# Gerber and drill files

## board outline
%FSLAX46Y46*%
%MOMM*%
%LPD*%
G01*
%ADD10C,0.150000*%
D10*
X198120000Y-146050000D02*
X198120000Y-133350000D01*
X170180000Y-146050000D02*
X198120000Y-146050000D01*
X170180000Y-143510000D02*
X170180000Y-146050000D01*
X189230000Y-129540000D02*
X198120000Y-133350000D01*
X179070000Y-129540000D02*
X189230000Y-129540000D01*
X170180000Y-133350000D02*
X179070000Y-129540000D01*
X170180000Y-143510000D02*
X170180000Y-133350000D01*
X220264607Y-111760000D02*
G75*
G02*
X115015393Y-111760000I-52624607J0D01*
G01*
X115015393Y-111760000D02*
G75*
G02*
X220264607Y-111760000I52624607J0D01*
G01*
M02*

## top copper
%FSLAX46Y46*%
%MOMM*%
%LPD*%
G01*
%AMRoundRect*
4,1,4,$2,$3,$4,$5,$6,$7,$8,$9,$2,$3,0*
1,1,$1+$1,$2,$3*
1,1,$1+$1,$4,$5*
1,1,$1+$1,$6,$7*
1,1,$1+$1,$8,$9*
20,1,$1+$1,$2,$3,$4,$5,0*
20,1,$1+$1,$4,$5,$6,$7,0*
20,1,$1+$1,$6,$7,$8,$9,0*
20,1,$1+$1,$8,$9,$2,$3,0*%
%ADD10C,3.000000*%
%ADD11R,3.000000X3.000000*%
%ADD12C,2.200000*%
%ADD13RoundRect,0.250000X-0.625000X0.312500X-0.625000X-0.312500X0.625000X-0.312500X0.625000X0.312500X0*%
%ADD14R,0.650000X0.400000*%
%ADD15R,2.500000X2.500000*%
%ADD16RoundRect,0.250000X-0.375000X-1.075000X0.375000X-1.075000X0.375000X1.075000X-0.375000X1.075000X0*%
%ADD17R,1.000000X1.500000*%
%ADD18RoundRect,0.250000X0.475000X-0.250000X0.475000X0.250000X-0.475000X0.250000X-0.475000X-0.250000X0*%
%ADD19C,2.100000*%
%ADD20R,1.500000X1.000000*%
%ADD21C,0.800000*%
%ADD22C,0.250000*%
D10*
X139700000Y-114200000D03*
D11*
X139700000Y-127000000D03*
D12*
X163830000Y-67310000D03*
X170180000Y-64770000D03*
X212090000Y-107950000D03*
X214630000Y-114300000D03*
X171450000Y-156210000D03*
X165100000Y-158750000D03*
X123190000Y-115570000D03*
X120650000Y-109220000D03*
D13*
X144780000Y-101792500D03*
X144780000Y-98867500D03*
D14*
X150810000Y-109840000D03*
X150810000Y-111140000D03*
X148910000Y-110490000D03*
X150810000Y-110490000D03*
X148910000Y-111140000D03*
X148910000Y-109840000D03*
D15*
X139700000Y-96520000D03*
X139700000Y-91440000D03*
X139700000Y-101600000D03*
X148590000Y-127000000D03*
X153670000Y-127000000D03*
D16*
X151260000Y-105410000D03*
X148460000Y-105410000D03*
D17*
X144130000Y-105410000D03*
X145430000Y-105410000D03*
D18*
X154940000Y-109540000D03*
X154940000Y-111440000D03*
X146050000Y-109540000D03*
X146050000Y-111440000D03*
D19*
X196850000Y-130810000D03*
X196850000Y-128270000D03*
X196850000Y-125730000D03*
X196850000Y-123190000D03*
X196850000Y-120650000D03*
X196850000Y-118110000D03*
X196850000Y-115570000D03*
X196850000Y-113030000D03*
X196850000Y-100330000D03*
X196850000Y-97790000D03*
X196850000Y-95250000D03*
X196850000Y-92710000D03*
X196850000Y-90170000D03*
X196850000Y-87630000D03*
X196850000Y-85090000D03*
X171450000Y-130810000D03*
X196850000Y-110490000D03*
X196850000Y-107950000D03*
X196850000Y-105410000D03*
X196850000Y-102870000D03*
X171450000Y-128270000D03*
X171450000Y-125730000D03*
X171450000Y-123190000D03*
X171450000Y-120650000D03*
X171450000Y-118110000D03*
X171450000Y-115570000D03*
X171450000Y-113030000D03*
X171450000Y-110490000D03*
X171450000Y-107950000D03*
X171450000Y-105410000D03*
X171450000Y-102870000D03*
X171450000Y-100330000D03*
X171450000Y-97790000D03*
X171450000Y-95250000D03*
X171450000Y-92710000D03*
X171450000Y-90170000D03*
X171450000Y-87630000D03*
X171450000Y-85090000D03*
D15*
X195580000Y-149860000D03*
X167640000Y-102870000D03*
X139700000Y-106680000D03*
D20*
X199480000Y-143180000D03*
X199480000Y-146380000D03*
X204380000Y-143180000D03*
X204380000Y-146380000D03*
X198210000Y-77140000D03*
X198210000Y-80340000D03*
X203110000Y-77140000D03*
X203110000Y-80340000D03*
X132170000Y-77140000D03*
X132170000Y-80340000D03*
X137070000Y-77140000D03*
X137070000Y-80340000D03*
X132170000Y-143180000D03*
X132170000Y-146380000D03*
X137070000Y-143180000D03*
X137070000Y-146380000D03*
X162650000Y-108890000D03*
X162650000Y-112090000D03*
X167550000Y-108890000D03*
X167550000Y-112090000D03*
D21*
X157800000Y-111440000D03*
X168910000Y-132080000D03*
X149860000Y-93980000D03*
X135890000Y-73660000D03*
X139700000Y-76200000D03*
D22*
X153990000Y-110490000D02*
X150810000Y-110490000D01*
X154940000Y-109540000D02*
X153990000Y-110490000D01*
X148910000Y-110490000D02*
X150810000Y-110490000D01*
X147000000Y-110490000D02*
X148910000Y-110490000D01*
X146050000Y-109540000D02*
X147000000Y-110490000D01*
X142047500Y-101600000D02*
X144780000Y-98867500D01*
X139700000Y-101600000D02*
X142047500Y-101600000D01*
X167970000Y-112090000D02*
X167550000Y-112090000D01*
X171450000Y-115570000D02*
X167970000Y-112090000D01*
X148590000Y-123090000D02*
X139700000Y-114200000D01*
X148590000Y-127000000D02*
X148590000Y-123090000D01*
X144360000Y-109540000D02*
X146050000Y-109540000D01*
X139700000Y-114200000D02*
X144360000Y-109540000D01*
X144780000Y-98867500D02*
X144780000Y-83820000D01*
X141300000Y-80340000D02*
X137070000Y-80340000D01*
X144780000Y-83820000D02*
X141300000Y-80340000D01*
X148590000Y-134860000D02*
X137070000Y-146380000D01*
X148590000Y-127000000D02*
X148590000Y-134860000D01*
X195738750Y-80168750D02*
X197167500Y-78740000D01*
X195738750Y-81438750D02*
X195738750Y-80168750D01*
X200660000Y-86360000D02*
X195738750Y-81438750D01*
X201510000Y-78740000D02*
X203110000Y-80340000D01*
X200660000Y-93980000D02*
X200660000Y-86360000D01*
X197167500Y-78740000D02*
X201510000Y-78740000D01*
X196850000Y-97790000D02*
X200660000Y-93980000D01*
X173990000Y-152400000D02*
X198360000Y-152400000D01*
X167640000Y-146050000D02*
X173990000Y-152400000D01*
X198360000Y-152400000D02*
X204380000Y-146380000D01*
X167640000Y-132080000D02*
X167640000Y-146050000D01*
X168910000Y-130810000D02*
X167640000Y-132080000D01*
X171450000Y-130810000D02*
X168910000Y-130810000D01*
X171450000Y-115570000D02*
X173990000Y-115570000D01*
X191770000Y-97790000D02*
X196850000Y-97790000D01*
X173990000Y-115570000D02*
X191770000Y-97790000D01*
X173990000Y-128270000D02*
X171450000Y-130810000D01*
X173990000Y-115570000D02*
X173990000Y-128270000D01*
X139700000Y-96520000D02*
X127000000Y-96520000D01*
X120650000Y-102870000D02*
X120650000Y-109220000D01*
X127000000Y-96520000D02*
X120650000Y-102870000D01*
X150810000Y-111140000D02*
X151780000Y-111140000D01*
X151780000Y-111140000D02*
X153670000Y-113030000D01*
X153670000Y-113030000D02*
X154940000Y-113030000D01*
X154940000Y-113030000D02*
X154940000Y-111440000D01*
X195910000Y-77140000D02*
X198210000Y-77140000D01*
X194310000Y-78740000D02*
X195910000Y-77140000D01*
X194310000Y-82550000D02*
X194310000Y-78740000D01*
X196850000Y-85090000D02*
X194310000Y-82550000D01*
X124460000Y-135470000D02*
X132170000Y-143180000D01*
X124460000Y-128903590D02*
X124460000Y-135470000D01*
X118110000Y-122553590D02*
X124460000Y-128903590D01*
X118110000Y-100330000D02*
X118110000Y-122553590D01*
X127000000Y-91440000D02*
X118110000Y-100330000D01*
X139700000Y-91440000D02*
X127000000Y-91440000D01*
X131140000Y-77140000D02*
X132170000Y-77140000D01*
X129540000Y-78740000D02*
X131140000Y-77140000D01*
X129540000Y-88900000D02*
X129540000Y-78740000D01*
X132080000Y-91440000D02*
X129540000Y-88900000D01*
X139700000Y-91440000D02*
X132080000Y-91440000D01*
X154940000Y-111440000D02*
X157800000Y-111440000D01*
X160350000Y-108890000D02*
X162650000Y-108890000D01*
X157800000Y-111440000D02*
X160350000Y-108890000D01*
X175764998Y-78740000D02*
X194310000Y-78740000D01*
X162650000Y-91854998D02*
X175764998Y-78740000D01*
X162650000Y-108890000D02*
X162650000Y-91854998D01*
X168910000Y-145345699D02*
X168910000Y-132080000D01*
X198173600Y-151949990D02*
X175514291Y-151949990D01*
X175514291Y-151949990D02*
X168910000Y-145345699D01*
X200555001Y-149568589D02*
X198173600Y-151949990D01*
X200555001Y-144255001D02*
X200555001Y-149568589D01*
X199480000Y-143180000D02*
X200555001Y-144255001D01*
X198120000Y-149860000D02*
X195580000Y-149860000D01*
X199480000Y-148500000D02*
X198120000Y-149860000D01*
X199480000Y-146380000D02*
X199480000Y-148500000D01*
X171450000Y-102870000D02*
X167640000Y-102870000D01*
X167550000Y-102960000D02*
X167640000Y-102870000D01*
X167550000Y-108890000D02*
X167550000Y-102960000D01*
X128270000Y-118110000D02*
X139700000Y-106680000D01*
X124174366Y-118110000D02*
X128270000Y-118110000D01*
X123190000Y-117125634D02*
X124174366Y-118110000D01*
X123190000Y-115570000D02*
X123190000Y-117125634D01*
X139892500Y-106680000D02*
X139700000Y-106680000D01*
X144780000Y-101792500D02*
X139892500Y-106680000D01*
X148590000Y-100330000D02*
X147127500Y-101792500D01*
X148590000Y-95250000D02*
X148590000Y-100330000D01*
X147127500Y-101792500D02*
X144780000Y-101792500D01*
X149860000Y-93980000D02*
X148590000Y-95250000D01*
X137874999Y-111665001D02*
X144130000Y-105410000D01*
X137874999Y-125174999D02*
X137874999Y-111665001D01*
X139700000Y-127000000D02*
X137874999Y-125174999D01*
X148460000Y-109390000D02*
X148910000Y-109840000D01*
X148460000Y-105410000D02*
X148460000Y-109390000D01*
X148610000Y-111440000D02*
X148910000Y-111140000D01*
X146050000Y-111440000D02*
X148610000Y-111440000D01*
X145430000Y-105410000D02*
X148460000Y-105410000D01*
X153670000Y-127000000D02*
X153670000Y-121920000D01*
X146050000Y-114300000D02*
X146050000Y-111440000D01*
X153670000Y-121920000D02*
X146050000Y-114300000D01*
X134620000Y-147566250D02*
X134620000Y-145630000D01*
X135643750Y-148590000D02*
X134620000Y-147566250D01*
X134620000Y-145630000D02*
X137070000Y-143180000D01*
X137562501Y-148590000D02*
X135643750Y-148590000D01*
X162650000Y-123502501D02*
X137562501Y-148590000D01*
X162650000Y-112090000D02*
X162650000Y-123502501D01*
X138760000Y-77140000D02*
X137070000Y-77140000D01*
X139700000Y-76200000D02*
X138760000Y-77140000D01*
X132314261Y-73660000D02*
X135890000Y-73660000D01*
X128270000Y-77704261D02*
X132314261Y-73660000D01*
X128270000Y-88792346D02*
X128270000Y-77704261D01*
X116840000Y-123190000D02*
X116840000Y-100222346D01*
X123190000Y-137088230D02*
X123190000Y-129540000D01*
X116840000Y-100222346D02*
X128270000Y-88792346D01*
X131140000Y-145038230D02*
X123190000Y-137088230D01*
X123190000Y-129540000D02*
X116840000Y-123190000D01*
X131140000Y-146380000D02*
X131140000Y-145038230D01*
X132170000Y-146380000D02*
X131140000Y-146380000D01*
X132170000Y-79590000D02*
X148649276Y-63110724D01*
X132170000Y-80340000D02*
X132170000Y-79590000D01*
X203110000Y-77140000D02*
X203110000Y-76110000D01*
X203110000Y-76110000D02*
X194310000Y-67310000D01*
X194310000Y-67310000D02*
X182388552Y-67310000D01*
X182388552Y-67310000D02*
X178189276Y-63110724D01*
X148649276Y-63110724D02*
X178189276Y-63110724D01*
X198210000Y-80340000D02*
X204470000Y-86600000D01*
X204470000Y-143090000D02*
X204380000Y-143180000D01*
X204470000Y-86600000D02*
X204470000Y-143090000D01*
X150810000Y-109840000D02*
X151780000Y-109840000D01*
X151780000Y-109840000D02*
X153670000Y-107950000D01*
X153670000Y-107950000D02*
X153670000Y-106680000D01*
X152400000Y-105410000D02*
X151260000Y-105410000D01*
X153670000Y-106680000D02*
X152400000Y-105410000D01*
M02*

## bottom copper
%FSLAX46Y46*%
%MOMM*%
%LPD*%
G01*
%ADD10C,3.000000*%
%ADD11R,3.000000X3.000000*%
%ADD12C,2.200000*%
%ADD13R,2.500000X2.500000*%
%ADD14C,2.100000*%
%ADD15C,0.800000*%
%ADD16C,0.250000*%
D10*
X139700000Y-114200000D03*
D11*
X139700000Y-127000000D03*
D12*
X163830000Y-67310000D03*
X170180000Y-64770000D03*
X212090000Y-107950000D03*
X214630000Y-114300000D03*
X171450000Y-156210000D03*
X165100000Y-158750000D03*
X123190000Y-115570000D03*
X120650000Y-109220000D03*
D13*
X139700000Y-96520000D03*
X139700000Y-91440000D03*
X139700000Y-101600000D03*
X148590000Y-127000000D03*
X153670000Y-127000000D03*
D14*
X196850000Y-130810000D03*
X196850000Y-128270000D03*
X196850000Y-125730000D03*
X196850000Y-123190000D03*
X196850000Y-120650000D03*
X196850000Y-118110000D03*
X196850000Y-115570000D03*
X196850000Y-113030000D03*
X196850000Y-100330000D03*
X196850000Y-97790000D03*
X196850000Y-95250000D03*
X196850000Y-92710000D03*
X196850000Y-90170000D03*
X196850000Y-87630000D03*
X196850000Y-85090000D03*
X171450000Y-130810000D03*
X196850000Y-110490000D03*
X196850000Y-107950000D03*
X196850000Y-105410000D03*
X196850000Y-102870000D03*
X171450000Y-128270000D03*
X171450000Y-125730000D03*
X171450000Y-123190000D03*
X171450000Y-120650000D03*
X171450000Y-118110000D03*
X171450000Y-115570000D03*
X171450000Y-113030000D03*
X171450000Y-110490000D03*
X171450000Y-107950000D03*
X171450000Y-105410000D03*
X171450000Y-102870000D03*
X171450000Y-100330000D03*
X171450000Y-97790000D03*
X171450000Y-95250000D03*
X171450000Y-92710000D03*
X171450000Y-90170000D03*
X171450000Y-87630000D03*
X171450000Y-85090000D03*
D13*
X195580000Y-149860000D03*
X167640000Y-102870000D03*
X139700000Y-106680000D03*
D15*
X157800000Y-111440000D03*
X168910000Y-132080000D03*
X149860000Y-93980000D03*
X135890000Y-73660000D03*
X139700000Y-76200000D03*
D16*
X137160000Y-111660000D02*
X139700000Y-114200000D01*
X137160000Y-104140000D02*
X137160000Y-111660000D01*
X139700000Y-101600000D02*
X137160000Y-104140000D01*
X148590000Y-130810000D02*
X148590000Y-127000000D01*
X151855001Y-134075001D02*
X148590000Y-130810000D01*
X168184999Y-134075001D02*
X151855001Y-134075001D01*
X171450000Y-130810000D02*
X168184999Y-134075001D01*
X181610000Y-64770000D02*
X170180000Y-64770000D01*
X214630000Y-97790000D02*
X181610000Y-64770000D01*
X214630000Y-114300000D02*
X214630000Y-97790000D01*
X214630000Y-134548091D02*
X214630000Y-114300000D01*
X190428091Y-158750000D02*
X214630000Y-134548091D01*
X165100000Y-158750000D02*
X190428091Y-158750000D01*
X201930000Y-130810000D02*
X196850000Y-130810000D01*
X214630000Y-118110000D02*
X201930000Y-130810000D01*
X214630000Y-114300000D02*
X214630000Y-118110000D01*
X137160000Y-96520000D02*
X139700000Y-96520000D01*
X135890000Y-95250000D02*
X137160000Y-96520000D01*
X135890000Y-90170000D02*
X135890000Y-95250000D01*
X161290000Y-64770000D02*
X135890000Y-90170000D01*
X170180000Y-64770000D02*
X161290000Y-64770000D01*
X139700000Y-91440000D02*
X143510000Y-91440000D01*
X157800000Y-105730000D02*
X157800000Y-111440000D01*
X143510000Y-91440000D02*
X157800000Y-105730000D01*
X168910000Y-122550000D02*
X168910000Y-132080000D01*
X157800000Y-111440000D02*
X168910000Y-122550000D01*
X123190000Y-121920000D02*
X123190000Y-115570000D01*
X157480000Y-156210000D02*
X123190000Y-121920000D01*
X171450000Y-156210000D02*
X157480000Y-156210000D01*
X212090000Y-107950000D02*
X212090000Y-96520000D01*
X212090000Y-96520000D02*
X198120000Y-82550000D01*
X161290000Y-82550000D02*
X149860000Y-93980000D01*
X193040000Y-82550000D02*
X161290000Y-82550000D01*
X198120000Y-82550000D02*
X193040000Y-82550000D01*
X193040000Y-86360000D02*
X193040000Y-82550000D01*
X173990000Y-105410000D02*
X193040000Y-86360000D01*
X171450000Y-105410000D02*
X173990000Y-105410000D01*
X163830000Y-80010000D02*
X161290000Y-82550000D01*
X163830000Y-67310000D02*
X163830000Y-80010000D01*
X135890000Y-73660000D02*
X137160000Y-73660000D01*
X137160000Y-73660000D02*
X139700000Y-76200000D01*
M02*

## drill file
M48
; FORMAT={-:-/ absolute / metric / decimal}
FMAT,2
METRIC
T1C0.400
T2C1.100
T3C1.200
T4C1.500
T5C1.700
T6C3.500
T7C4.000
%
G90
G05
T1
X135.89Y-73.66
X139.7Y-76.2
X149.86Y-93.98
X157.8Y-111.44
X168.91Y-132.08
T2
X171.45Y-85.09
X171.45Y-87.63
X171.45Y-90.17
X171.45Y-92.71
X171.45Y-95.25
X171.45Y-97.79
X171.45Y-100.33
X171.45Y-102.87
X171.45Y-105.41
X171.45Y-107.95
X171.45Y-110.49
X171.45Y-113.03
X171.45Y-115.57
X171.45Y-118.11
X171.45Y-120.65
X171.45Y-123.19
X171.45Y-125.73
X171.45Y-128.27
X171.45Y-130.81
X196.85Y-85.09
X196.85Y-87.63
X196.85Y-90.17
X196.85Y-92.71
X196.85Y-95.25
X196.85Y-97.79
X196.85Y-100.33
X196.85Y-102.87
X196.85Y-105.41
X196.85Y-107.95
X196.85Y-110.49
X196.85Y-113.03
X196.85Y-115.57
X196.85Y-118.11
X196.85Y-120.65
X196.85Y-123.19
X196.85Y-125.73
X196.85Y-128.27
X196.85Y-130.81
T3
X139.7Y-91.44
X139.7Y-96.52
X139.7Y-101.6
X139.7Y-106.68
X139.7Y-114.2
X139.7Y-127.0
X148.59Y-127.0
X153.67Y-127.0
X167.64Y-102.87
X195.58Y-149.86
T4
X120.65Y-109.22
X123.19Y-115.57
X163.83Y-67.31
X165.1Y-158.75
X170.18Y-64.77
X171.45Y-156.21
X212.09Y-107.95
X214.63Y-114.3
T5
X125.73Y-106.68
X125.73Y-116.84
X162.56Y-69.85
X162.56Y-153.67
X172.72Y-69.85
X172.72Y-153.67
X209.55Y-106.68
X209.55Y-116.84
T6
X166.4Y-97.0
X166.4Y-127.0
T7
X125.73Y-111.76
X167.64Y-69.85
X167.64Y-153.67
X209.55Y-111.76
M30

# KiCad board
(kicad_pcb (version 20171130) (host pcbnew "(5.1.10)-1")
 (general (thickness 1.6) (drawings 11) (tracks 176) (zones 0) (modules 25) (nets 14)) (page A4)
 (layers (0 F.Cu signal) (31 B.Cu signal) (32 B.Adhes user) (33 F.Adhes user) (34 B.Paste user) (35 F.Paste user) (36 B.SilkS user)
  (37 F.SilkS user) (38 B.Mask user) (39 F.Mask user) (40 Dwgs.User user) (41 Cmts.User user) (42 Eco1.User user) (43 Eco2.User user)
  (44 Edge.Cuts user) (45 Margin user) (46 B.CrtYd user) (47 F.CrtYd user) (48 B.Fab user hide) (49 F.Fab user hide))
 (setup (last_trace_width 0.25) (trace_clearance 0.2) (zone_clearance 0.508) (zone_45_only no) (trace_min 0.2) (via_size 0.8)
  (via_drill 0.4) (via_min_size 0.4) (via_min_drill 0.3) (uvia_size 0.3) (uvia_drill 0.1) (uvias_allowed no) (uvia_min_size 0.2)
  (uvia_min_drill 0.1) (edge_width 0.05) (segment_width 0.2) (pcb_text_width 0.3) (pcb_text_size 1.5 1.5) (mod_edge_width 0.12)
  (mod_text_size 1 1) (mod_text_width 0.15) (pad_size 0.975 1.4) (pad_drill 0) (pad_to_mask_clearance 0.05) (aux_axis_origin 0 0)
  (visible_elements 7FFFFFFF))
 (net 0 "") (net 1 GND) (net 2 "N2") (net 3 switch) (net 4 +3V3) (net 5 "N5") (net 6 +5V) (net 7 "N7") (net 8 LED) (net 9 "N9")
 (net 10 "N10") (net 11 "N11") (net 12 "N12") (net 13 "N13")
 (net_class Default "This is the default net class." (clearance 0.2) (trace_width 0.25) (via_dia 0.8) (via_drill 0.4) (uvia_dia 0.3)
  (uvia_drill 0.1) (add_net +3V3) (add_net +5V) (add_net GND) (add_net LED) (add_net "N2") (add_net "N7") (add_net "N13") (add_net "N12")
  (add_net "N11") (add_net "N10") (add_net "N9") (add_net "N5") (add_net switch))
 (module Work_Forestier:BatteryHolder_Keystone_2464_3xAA (layer B.Cu) (at 139.7 127)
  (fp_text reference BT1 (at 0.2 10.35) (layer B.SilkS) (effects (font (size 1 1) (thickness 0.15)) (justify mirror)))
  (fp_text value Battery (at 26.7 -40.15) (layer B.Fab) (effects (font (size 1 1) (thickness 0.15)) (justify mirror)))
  (pad "" np_thru_hole circle (at 26.7 -30) (size 3.5 3.5) (drill 3.5) (layers *.Cu *.Mask))
  (pad "" np_thru_hole circle (at 26.7 0) (size 3.5 3.5) (drill 3.5) (layers *.Cu *.Mask))
  (pad 2 thru_hole circle (at 0 -12.8) (size 3 3) (drill 1.2) (layers *.Cu *.Mask) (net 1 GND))
  (pad 1 thru_hole rect (at 0 0) (size 3 3) (drill 1.2) (layers *.Cu *.Mask) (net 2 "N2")))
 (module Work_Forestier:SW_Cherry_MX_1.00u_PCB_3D (layer F.Cu) (at 170.18 64.77)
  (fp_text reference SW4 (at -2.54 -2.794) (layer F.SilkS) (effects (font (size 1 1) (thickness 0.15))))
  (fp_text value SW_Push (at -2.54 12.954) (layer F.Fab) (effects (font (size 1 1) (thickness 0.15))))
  (pad "" np_thru_hole circle (at 2.54 5.08) (size 1.7 1.7) (drill 1.7) (layers *.Cu *.Mask))
  (pad "" np_thru_hole circle (at -7.62 5.08) (size 1.7 1.7) (drill 1.7) (layers *.Cu *.Mask))
  (pad "" np_thru_hole circle (at -2.54 5.08) (size 4 4) (drill 4) (layers *.Cu *.Mask))
  (pad 2 thru_hole circle (at -6.35 2.54) (size 2.2 2.2) (drill 1.5) (layers *.Cu *.Mask) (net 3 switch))
  (pad 1 thru_hole circle (at 0 0) (size 2.2 2.2) (drill 1.5) (layers *.Cu *.Mask) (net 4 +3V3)))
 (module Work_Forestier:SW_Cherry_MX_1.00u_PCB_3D (layer F.Cu) (at 214.63 114.3 270)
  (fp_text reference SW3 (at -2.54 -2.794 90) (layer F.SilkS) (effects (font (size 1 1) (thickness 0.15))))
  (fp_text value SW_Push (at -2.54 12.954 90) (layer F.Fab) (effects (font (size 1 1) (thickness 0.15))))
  (pad "" np_thru_hole circle (at 2.54 5.08 270) (size 1.7 1.7) (drill 1.7) (layers *.Cu *.Mask))
  (pad "" np_thru_hole circle (at -7.62 5.08 270) (size 1.7 1.7) (drill 1.7) (layers *.Cu *.Mask))
  (pad "" np_thru_hole circle (at -2.54 5.08 270) (size 4 4) (drill 4) (layers *.Cu *.Mask))
  (pad 2 thru_hole circle (at -6.35 2.54 270) (size 2.2 2.2) (drill 1.5) (layers *.Cu *.Mask) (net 3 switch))
  (pad 1 thru_hole circle (at 0 0 270) (size 2.2 2.2) (drill 1.5) (layers *.Cu *.Mask) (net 4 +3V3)))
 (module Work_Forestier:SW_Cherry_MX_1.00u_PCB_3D (layer F.Cu) (at 165.1 158.75 180)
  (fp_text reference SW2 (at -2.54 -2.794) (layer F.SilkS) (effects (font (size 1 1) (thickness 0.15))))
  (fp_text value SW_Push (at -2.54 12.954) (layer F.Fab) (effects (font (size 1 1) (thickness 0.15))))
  (pad "" np_thru_hole circle (at 2.54 5.08 180) (size 1.7 1.7) (drill 1.7) (layers *.Cu *.Mask))
  (pad "" np_thru_hole circle (at -7.62 5.08 180) (size 1.7 1.7) (drill 1.7) (layers *.Cu *.Mask))
  (pad "" np_thru_hole circle (at -2.54 5.08 180) (size 4 4) (drill 4) (layers *.Cu *.Mask))
  (pad 2 thru_hole circle (at -6.35 2.54 180) (size 2.2 2.2) (drill 1.5) (layers *.Cu *.Mask) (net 3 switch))
  (pad 1 thru_hole circle (at 0 0 180) (size 2.2 2.2) (drill 1.5) (layers *.Cu *.Mask) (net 4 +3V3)))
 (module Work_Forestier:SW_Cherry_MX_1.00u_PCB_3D (layer F.Cu) (at 120.65 109.22 90)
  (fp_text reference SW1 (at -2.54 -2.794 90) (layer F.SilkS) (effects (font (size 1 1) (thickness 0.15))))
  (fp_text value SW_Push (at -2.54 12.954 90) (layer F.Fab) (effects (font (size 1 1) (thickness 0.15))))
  (pad "" np_thru_hole circle (at 2.54 5.08 90) (size 1.7 1.7) (drill 1.7) (layers *.Cu *.Mask))
  (pad "" np_thru_hole circle (at -7.62 5.08 90) (size 1.7 1.7) (drill 1.7) (layers *.Cu *.Mask))
  (pad "" np_thru_hole circle (at -2.54 5.08 90) (size 4 4) (drill 4) (layers *.Cu *.Mask))
  (pad 2 thru_hole circle (at -6.35 2.54 90) (size 2.2 2.2) (drill 1.5) (layers *.Cu *.Mask) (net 3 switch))
  (pad 1 thru_hole circle (at 0 0 90) (size 2.2 2.2) (drill 1.5) (layers *.Cu *.Mask) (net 4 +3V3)))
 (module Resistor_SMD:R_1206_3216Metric (layer F.Cu) (at 144.78 100.33 270)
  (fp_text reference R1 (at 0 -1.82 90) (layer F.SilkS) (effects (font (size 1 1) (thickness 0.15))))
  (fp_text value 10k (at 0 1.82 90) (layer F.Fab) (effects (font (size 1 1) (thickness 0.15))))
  (pad 2 smd roundrect (at 1.4625 0 270) (size 1.125 1.75) (layers F.Cu F.Paste F.Mask) (roundrect_rratio 0.222222) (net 3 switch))
  (pad 1 smd roundrect (at -1.4625 0 270) (size 1.125 1.75) (layers F.Cu F.Paste F.Mask) (roundrect_rratio 0.222222) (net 1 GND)))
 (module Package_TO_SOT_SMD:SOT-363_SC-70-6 (layer F.Cu) (at 149.86 110.49)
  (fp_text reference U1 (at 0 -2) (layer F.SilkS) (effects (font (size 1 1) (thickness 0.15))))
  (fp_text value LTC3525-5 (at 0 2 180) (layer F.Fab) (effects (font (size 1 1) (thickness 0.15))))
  (pad 6 smd rect (at 0.95 -0.65) (size 0.65 0.4) (layers F.Cu F.Paste F.Mask) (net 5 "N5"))
  (pad 4 smd rect (at 0.95 0.65) (size 0.65 0.4) (layers F.Cu F.Paste F.Mask) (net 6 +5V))
  (pad 2 smd rect (at -0.95 0) (size 0.65 0.4) (layers F.Cu F.Paste F.Mask) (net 1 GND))
  (pad 5 smd rect (at 0.95 0) (size 0.65 0.4) (layers F.Cu F.Paste F.Mask) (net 1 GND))
  (pad 3 smd rect (at -0.95 0.65) (size 0.65 0.4) (layers F.Cu F.Paste F.Mask) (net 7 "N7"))
  (pad 1 smd rect (at -0.95 -0.65) (size 0.65 0.4) (layers F.Cu F.Paste F.Mask) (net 7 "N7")))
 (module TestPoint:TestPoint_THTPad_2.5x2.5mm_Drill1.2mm (layer F.Cu) (at 139.7 96.52)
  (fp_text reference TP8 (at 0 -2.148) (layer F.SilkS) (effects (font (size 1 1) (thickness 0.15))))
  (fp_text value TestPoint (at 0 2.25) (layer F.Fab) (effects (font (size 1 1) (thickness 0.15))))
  (pad 1 thru_hole rect (at 0 0) (size 2.5 2.5) (drill 1.2) (layers *.Cu *.Mask) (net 4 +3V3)))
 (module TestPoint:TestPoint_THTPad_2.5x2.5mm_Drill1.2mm (layer F.Cu) (at 139.7 91.44)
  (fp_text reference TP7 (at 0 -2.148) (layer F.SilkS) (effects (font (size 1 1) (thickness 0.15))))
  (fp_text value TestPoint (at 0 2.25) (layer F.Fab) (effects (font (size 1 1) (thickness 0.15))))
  (pad 1 thru_hole rect (at 0 0) (size 2.5 2.5) (drill 1.2) (layers *.Cu *.Mask) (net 6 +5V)))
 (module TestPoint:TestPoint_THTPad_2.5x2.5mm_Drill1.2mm (layer F.Cu) (at 139.7 101.6)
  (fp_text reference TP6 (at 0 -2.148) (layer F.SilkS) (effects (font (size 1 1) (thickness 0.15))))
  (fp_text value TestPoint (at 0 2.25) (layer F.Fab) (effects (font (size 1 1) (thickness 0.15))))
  (pad 1 thru_hole rect (at 0 0) (size 2.5 2.5) (drill 1.2) (layers *.Cu *.Mask) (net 1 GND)))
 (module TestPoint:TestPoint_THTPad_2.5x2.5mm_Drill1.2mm (layer F.Cu) (at 148.59 127)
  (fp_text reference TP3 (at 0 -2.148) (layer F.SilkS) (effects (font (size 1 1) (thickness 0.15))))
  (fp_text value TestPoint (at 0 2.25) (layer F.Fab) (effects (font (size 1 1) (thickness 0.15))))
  (pad 1 thru_hole rect (at 0 0) (size 2.5 2.5) (drill 1.2) (layers *.Cu *.Mask) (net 1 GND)))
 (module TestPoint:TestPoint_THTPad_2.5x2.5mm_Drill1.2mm (layer F.Cu) (at 153.67 127)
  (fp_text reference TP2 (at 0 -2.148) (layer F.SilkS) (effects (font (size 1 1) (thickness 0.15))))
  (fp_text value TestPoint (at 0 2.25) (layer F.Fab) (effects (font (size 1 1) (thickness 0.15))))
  (pad 1 thru_hole rect (at 0 0) (size 2.5 2.5) (drill 1.2) (layers *.Cu *.Mask) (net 7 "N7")))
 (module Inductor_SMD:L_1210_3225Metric (layer F.Cu) (at 149.86 105.41)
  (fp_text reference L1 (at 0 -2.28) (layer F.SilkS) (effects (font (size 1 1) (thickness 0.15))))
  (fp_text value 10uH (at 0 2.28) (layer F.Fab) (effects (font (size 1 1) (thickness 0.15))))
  (pad 2 smd roundrect (at 1.4 0) (size 1.25 2.65) (layers F.Cu F.Paste F.Mask) (roundrect_rratio 0.2) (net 5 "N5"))
  (pad 1 smd roundrect (at -1.4 0) (size 1.25 2.65) (layers F.Cu F.Paste F.Mask) (roundrect_rratio 0.2) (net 7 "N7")))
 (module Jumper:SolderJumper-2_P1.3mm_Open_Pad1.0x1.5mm (layer F.Cu) (at 144.78 105.41)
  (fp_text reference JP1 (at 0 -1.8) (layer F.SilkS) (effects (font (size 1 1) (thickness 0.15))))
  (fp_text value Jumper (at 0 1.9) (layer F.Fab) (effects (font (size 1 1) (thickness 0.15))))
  (pad 1 smd rect (at -0.65 0) (size 1 1.5) (layers F.Cu F.Mask) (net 2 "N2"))
  (pad 2 smd rect (at 0.65 0) (size 1 1.5) (layers F.Cu F.Mask) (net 7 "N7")))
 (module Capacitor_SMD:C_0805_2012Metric (layer F.Cu) (at 154.94 110.49 90)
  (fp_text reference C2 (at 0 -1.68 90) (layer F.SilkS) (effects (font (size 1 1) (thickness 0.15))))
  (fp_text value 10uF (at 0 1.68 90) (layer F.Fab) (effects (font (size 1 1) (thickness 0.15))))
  (pad 2 smd roundrect (at 0.95 0 90) (size 1 1.45) (layers F.Cu F.Paste F.Mask) (roundrect_rratio 0.25) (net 1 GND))
  (pad 1 smd roundrect (at -0.95 0 90) (size 1 1.45) (layers F.Cu F.Paste F.Mask) (roundrect_rratio 0.25) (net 6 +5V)))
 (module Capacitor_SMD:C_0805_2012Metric (layer F.Cu) (at 146.05 110.49 90)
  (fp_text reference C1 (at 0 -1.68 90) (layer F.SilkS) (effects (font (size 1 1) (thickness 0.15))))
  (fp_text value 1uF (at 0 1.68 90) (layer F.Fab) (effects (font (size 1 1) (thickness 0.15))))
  (pad 2 smd roundrect (at 0.95 0 90) (size 1 1.45) (layers F.Cu F.Paste F.Mask) (roundrect_rratio 0.25) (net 1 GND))
  (pad 1 smd roundrect (at -0.95 0 90) (size 1 1.45) (layers F.Cu F.Paste F.Mask) (roundrect_rratio 0.25) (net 7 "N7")))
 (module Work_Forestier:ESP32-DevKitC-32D (layer F.Cu) (at 198.12 139.7 90)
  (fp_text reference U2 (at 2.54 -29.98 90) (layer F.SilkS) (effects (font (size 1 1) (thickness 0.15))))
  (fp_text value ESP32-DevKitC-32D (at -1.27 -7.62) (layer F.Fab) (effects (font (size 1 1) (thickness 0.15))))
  (pad 3V3 thru_hole circle (at 8.89 -1.27 90) (size 2.1 2.1) (drill 1.1) (layers *.Cu *.Mask) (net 4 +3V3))
  (pad EN thru_hole circle (at 11.43 -1.27 90) (size 2.1 2.1) (drill 1.1) (layers *.Cu *.Mask))
  (pad SVP thru_hole circle (at 13.97 -1.27 90) (size 2.1 2.1) (drill 1.1) (layers *.Cu *.Mask))
  (pad SVN thru_hole circle (at 16.51 -1.27 90) (size 2.1 2.1) (drill 1.1) (layers *.Cu *.Mask))
  (pad IO34 thru_hole circle (at 19.05 -1.27 90) (size 2.1 2.1) (drill 1.1) (layers *.Cu *.Mask))
  (pad IO35 thru_hole circle (at 21.59 -1.27 90) (size 2.1 2.1) (drill 1.1) (layers *.Cu *.Mask))
  (pad IO32 thru_hole circle (at 24.13 -1.27 90) (size 2.1 2.1) (drill 1.1) (layers *.Cu *.Mask))
  (pad IO33 thru_hole circle (at 26.67 -1.27 90) (size 2.1 2.1) (drill 1.1) (layers *.Cu *.Mask))
  (pad IO12 thru_hole circle (at 39.37 -1.27 90) (size 2.1 2.1) (drill 1.1) (layers *.Cu *.Mask))
  (pad GND0 thru_hole circle (at 41.91 -1.27 90) (size 2.1 2.1) (drill 1.1) (layers *.Cu *.Mask) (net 1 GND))
  (pad IO13 thru_hole circle (at 44.45 -1.27 90) (size 2.1 2.1) (drill 1.1) (layers *.Cu *.Mask))
  (pad SD2 thru_hole circle (at 46.99 -1.27 90) (size 2.1 2.1) (drill 1.1) (layers *.Cu *.Mask))
  (pad SD3 thru_hole circle (at 49.53 -1.27 90) (size 2.1 2.1) (drill 1.1) (layers *.Cu *.Mask))
  (pad CMD thru_hole circle (at 52.07 -1.27 90) (size 2.1 2.1) (drill 1.1) (layers *.Cu *.Mask))
  (pad 5V thru_hole circle (at 54.61 -1.27 90) (size 2.1 2.1) (drill 1.1) (layers *.Cu *.Mask) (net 6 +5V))
  (pad GND1 thru_hole circle (at 8.89 -26.67 90) (size 2.1 2.1) (drill 1.1) (layers *.Cu *.Mask) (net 1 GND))
  (pad IO25 thru_hole circle (at 29.21 -1.27 90) (size 2.1 2.1) (drill 1.1) (layers *.Cu *.Mask))
  (pad IO26 thru_hole circle (at 31.75 -1.27 90) (size 2.1 2.1) (drill 1.1) (layers *.Cu *.Mask))
  (pad IO27 thru_hole circle (at 34.29 -1.27 90) (size 2.1 2.1) (drill 1.1) (layers *.Cu *.Mask))
  (pad IO14 thru_hole circle (at 36.83 -1.27 90) (size 2.1 2.1) (drill 1.1) (layers *.Cu *.Mask))
  (pad IO23 thru_hole circle (at 11.43 -26.67 90) (size 2.1 2.1) (drill 1.1) (layers *.Cu *.Mask))
  (pad IO22 thru_hole circle (at 13.97 -26.67 90) (size 2.1 2.1) (drill 1.1) (layers *.Cu *.Mask))
  (pad TXD0 thru_hole circle (at 16.51 -26.67 90) (size 2.1 2.1) (drill 1.1) (layers *.Cu *.Mask))
  (pad RXD0 thru_hole circle (at 19.05 -26.67 90) (size 2.1 2.1) (drill 1.1) (layers *.Cu *.Mask))
  (pad IO21 thru_hole circle (at 21.59 -26.67 90) (size 2.1 2.1) (drill 1.1) (layers *.Cu *.Mask))
  (pad GND2 thru_hole circle (at 24.13 -26.67 90) (size 2.1 2.1) (drill 1.1) (layers *.Cu *.Mask) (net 1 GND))
  (pad IO19 thru_hole circle (at 26.67 -26.67 90) (size 2.1 2.1) (drill 1.1) (layers *.Cu *.Mask))
  (pad IO18 thru_hole circle (at 29.21 -26.67 90) (size 2.1 2.1) (drill 1.1) (layers *.Cu *.Mask))
  (pad IO5 thru_hole circle (at 31.75 -26.67 90) (size 2.1 2.1) (drill 1.1) (layers *.Cu *.Mask))
  (pad IO17 thru_hole circle (at 34.29 -26.67 90) (size 2.1 2.1) (drill 1.1) (layers *.Cu *.Mask) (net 3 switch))
  (pad IO16 thru_hole circle (at 36.83 -26.67 90) (size 2.1 2.1) (drill 1.1) (layers *.Cu *.Mask) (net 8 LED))
  (pad IO4 thru_hole circle (at 39.37 -26.67 90) (size 2.1 2.1) (drill 1.1) (layers *.Cu *.Mask))
  (pad IO0 thru_hole circle (at 41.91 -26.67 90) (size 2.1 2.1) (drill 1.1) (layers *.Cu *.Mask))
  (pad IO2 thru_hole circle (at 44.45 -26.67 90) (size 2.1 2.1) (drill 1.1) (layers *.Cu *.Mask))
  (pad IO15 thru_hole circle (at 46.99 -26.67 90) (size 2.1 2.1) (drill 1.1) (layers *.Cu *.Mask))
  (pad SD1 thru_hole circle (at 49.53 -26.67 90) (size 2.1 2.1) (drill 1.1) (layers *.Cu *.Mask))
  (pad SD0 thru_hole circle (at 52.07 -26.67 90) (size 2.1 2.1) (drill 1.1) (layers *.Cu *.Mask))
  (pad CLK thru_hole circle (at 54.61 -26.67 90) (size 2.1 2.1) (drill 1.1) (layers *.Cu *.Mask)))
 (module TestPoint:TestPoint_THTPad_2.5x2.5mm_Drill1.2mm (layer F.Cu) (at 195.58 149.86)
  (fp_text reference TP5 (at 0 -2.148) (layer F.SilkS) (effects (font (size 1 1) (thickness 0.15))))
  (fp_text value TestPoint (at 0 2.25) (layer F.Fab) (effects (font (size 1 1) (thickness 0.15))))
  (pad 1 thru_hole rect (at 0 0) (size 2.5 2.5) (drill 1.2) (layers *.Cu *.Mask) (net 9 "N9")))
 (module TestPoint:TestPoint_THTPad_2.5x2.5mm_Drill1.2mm (layer F.Cu) (at 167.64 102.87)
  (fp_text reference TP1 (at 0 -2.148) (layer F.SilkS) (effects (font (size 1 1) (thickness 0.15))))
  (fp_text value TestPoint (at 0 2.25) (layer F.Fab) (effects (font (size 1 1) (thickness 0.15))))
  (pad 1 thru_hole rect (at 0 0) (size 2.5 2.5) (drill 1.2) (layers *.Cu *.Mask) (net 8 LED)))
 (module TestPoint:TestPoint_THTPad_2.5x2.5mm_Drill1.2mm (layer F.Cu) (at 139.7 106.68)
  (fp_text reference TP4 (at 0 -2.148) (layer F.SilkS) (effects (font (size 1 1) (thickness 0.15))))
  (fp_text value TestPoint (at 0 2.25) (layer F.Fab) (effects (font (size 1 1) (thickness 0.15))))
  (pad 1 thru_hole rect (at 0 0) (size 2.5 2.5) (drill 1.2) (layers *.Cu *.Mask) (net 3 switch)))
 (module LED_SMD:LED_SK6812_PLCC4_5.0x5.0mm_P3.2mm (layer F.Cu) (at 201.93 144.78)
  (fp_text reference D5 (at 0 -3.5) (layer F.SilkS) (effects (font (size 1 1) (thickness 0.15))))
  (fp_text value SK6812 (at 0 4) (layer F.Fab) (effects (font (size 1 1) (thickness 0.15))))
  (pad 3 smd rect (at -2.45 -1.6) (size 1.5 1) (layers F.Cu F.Paste F.Mask) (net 6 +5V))
  (pad 4 smd rect (at -2.45 1.6) (size 1.5 1) (layers F.Cu F.Paste F.Mask) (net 9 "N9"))
  (pad 2 smd rect (at 2.45 -1.6) (size 1.5 1) (layers F.Cu F.Paste F.Mask) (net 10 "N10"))
  (pad 1 smd rect (at 2.45 1.6) (size 1.5 1) (layers F.Cu F.Paste F.Mask) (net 1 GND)))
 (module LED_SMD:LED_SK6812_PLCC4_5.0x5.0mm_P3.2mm (layer F.Cu) (at 200.66 78.74)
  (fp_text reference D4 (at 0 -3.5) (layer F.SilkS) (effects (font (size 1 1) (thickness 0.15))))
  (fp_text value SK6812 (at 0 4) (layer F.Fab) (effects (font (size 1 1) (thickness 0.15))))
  (pad 3 smd rect (at -2.45 -1.6) (size 1.5 1) (layers F.Cu F.Paste F.Mask) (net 6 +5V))
  (pad 4 smd rect (at -2.45 1.6) (size 1.5 1) (layers F.Cu F.Paste F.Mask) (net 10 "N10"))
  (pad 2 smd rect (at 2.45 -1.6) (size 1.5 1) (layers F.Cu F.Paste F.Mask) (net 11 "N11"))
  (pad 1 smd rect (at 2.45 1.6) (size 1.5 1) (layers F.Cu F.Paste F.Mask) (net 1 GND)))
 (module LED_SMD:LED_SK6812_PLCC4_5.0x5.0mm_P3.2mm (layer F.Cu) (at 134.62 78.74)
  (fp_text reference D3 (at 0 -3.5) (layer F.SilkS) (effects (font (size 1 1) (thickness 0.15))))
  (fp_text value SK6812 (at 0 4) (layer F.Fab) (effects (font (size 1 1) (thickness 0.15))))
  (pad 3 smd rect (at -2.45 -1.6) (size 1.5 1) (layers F.Cu F.Paste F.Mask) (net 6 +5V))
  (pad 4 smd rect (at -2.45 1.6) (size 1.5 1) (layers F.Cu F.Paste F.Mask) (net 11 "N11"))
  (pad 2 smd rect (at 2.45 -1.6) (size 1.5 1) (layers F.Cu F.Paste F.Mask) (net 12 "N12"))
  (pad 1 smd rect (at 2.45 1.6) (size 1.5 1) (layers F.Cu F.Paste F.Mask) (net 1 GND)))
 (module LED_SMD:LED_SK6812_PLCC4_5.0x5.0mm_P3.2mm (layer F.Cu) (at 134.62 144.78)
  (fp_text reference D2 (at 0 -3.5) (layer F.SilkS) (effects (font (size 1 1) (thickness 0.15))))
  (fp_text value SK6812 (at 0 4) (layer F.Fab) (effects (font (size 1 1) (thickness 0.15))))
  (pad 3 smd rect (at -2.45 -1.6) (size 1.5 1) (layers F.Cu F.Paste F.Mask) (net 6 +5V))
  (pad 4 smd rect (at -2.45 1.6) (size 1.5 1) (layers F.Cu F.Paste F.Mask) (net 12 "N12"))
  (pad 2 smd rect (at 2.45 -1.6) (size 1.5 1) (layers F.Cu F.Paste F.Mask) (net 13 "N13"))
  (pad 1 smd rect (at 2.45 1.6) (size 1.5 1) (layers F.Cu F.Paste F.Mask) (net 1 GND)))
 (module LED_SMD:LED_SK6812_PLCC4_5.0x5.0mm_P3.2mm (layer F.Cu) (at 165.1 110.49)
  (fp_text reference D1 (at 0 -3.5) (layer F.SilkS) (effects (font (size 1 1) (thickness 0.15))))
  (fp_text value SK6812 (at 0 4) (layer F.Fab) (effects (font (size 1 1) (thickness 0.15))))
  (pad 3 smd rect (at -2.45 -1.6) (size 1.5 1) (layers F.Cu F.Paste F.Mask) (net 6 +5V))
  (pad 4 smd rect (at -2.45 1.6) (size 1.5 1) (layers F.Cu F.Paste F.Mask) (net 13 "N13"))
  (pad 2 smd rect (at 2.45 -1.6) (size 1.5 1) (layers F.Cu F.Paste F.Mask) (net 8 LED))
  (pad 1 smd rect (at 2.45 1.6) (size 1.5 1) (layers F.Cu F.Paste F.Mask) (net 1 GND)))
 (gr_line (start 198.12 146.05) (end 198.12 133.35) (layer Edge.Cuts) (width 0.15))
 (gr_line (start 170.18 146.05) (end 198.12 146.05) (layer Edge.Cuts) (width 0.15))
 (gr_line (start 170.18 143.51) (end 170.18 146.05) (layer Edge.Cuts) (width 0.15))
 (gr_line (start 189.23 129.54) (end 198.12 133.35) (layer Edge.Cuts) (width 0.15))
 (gr_line (start 179.07 129.54) (end 189.23 129.54) (layer Edge.Cuts) (width 0.15))
 (gr_line (start 170.18 133.35) (end 179.07 129.54) (layer Edge.Cuts) (width 0.15))
 (gr_line (start 170.18 143.51) (end 170.18 133.35) (layer Edge.Cuts) (width 0.15))
 (gr_circle (center 167.64 111.76) (end 220.264607 111.76) (layer Edge.Cuts) (width 0.15))
 (segment (start 153.99 110.49) (end 150.81 110.49) (width 0.25) (layer F.Cu) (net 1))
 (segment (start 154.94 109.54) (end 153.99 110.49) (width 0.25) (layer F.Cu) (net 1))
 (segment (start 148.91 110.49) (end 150.81 110.49) (width 0.25) (layer F.Cu) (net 1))
 (segment (start 147 110.49) (end 148.91 110.49) (width 0.25) (layer F.Cu) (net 1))
 (segment (start 146.05 109.54) (end 147 110.49) (width 0.25) (layer F.Cu) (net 1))
 (segment (start 142.0475 101.6) (end 144.78 98.8675) (width 0.25) (layer F.Cu) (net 1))
 (segment (start 139.7 101.6) (end 142.0475 101.6) (width 0.25) (layer F.Cu) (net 1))
 (segment (start 167.97 112.09) (end 167.55 112.09) (width 0.25) (layer F.Cu) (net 1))
 (segment (start 171.45 115.57) (end 167.97 112.09) (width 0.25) (layer F.Cu) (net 1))
 (segment (start 148.59 123.09) (end 139.7 114.2) (width 0.25) (layer F.Cu) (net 1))
 (segment (start 148.59 127) (end 148.59 123.09) (width 0.25) (layer F.Cu) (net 1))
 (segment (start 144.36 109.54) (end 146.05 109.54) (width 0.25) (layer F.Cu) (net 1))
 (segment (start 139.7 114.2) (end 144.36 109.54) (width 0.25) (layer F.Cu) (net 1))
 (segment (start 144.78 98.8675) (end 144.78 83.82) (width 0.25) (layer F.Cu) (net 1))
 (segment (start 141.3 80.34) (end 137.07 80.34) (width 0.25) (layer F.Cu) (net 1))
 (segment (start 144.78 83.82) (end 141.3 80.34) (width 0.25) (layer F.Cu) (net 1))
 (segment (start 148.59 134.86) (end 137.07 146.38) (width 0.25) (layer F.Cu) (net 1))
 (segment (start 148.59 127) (end 148.59 134.86) (width 0.25) (layer F.Cu) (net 1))
 (segment (start 195.73875 80.16875) (end 197.1675 78.74) (width 0.25) (layer F.Cu) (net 1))
 (segment (start 195.73875 81.43875) (end 195.73875 80.16875) (width 0.25) (layer F.Cu) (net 1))
 (segment (start 200.66 86.36) (end 195.73875 81.43875) (width 0.25) (layer F.Cu) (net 1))
 (segment (start 201.51 78.74) (end 203.11 80.34) (width 0.25) (layer F.Cu) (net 1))
 (segment (start 200.66 93.98) (end 200.66 86.36) (width 0.25) (layer F.Cu) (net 1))
 (segment (start 197.1675 78.74) (end 201.51 78.74) (width 0.25) (layer F.Cu) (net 1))
 (segment (start 196.85 97.79) (end 200.66 93.98) (width 0.25) (layer F.Cu) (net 1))
 (segment (start 173.99 152.4) (end 198.36 152.4) (width 0.25) (layer F.Cu) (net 1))
 (segment (start 167.64 146.05) (end 173.99 152.4) (width 0.25) (layer F.Cu) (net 1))
 (segment (start 198.36 152.4) (end 204.38 146.38) (width 0.25) (layer F.Cu) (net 1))
 (segment (start 167.64 132.08) (end 167.64 146.05) (width 0.25) (layer F.Cu) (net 1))
 (segment (start 168.91 130.81) (end 167.64 132.08) (width 0.25) (layer F.Cu) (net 1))
 (segment (start 171.45 130.81) (end 168.91 130.81) (width 0.25) (layer F.Cu) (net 1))
 (segment (start 137.16 111.66) (end 139.7 114.2) (width 0.25) (layer B.Cu) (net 1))
 (segment (start 137.16 104.14) (end 137.16 111.66) (width 0.25) (layer B.Cu) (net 1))
 (segment (start 139.7 101.6) (end 137.16 104.14) (width 0.25) (layer B.Cu) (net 1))
 (segment (start 171.45 115.57) (end 173.99 115.57) (width 0.25) (layer F.Cu) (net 1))
 (segment (start 191.77 97.79) (end 196.85 97.79) (width 0.25) (layer F.Cu) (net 1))
 (segment (start 173.99 115.57) (end 191.77 97.79) (width 0.25) (layer F.Cu) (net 1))
 (segment (start 148.59 130.81) (end 148.59 127) (width 0.25) (layer B.Cu) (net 1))
 (segment (start 151.855001 134.075001) (end 148.59 130.81) (width 0.25) (layer B.Cu) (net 1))
 (segment (start 168.184999 134.075001) (end 151.855001 134.075001) (width 0.25) (layer B.Cu) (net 1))
 (segment (start 171.45 130.81) (end 168.184999 134.075001) (width 0.25) (layer B.Cu) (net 1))
 (segment (start 173.99 128.27) (end 171.45 130.81) (width 0.25) (layer F.Cu) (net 1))
 (segment (start 173.99 115.57) (end 173.99 128.27) (width 0.25) (layer F.Cu) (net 1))
 (segment (start 139.7 96.52) (end 127 96.52) (width 0.25) (layer F.Cu) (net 4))
 (segment (start 120.65 102.87) (end 120.65 109.22) (width 0.25) (layer F.Cu) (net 4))
 (segment (start 127 96.52) (end 120.65 102.87) (width 0.25) (layer F.Cu) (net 4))
 (segment (start 181.61 64.77) (end 170.18 64.77) (width 0.25) (layer B.Cu) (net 4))
 (segment (start 214.63 97.79) (end 181.61 64.77) (width 0.25) (layer B.Cu) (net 4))
 (segment (start 214.63 114.3) (end 214.63 97.79) (width 0.25) (layer B.Cu) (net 4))
 (segment (start 214.63 134.548091) (end 214.63 114.3) (width 0.25) (layer B.Cu) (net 4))
 (segment (start 190.428091 158.75) (end 214.63 134.548091) (width 0.25) (layer B.Cu) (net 4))
 (segment (start 165.1 158.75) (end 190.428091 158.75) (width 0.25) (layer B.Cu) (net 4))
 (segment (start 201.93 130.81) (end 196.85 130.81) (width 0.25) (layer B.Cu) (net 4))
 (segment (start 214.63 118.11) (end 201.93 130.81) (width 0.25) (layer B.Cu) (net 4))
 (segment (start 214.63 114.3) (end 214.63 118.11) (width 0.25) (layer B.Cu) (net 4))
 (segment (start 137.16 96.52) (end 139.7 96.52) (width 0.25) (layer B.Cu) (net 4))
 (segment (start 135.89 95.25) (end 137.16 96.52) (width 0.25) (layer B.Cu) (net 4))
 (segment (start 135.89 90.17) (end 135.89 95.25) (width 0.25) (layer B.Cu) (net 4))
 (segment (start 161.29 64.77) (end 135.89 90.17) (width 0.25) (layer B.Cu) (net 4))
 (segment (start 170.18 64.77) (end 161.29 64.77) (width 0.25) (layer B.Cu) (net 4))
 (segment (start 150.81 111.14) (end 151.78 111.14) (width 0.25) (layer F.Cu) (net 6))
 (segment (start 151.78 111.14) (end 153.67 113.03) (width 0.25) (layer F.Cu) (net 6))
 (segment (start 153.67 113.03) (end 154.94 113.03) (width 0.25) (layer F.Cu) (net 6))
 (segment (start 154.94 113.03) (end 154.94 111.44) (width 0.25) (layer F.Cu) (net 6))
 (segment (start 195.91 77.14) (end 198.21 77.14) (width 0.25) (layer F.Cu) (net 6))
 (segment (start 194.31 78.74) (end 195.91 77.14) (width 0.25) (layer F.Cu) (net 6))
 (segment (start 194.31 82.55) (end 194.31 78.74) (width 0.25) (layer F.Cu) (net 6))
 (segment (start 196.85 85.09) (end 194.31 82.55) (width 0.25) (layer F.Cu) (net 6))
 (segment (start 124.46 135.47) (end 132.17 143.18) (width 0.25) (layer F.Cu) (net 6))
 (segment (start 124.46 128.90359) (end 124.46 135.47) (width 0.25) (layer F.Cu) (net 6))
 (segment (start 118.11 122.55359) (end 124.46 128.90359) (width 0.25) (layer F.Cu) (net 6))
 (segment (start 118.11 100.33) (end 118.11 122.55359) (width 0.25) (layer F.Cu) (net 6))
 (segment (start 127 91.44) (end 118.11 100.33) (width 0.25) (layer F.Cu) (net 6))
 (segment (start 139.7 91.44) (end 127 91.44) (width 0.25) (layer F.Cu) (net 6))
 (segment (start 131.14 77.14) (end 132.17 77.14) (width 0.25) (layer F.Cu) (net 6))
 (segment (start 129.54 78.74) (end 131.14 77.14) (width 0.25) (layer F.Cu) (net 6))
 (segment (start 129.54 88.9) (end 129.54 78.74) (width 0.25) (layer F.Cu) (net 6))
 (segment (start 132.08 91.44) (end 129.54 88.9) (width 0.25) (layer F.Cu) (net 6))
 (segment (start 139.7 91.44) (end 132.08 91.44) (width 0.25) (layer F.Cu) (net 6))
 (segment (start 154.94 111.44) (end 157.8 111.44) (width 0.25) (layer F.Cu) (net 6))
 (segment (start 160.35 108.89) (end 162.65 108.89) (width 0.25) (layer F.Cu) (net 6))
 (segment (start 157.8 111.44) (end 160.35 108.89) (width 0.25) (layer F.Cu) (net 6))
 (via (at 157.8 111.44) (size 0.8) (drill 0.4) (layers F.Cu B.Cu) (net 6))
 (segment (start 139.7 91.44) (end 143.51 91.44) (width 0.25) (layer B.Cu) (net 6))
 (segment (start 157.8 105.73) (end 157.8 111.44) (width 0.25) (layer B.Cu) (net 6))
 (segment (start 143.51 91.44) (end 157.8 105.73) (width 0.25) (layer B.Cu) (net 6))
 (segment (start 175.764998 78.74) (end 194.31 78.74) (width 0.25) (layer F.Cu) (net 6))
 (segment (start 162.65 91.854998) (end 175.764998 78.74) (width 0.25) (layer F.Cu) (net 6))
 (segment (start 162.65 108.89) (end 162.65 91.854998) (width 0.25) (layer F.Cu) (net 6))
 (segment (start 168.91 122.55) (end 168.91 132.08) (width 0.25) (layer B.Cu) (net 6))
 (segment (start 168.91 145.345699) (end 168.91 132.08) (width 0.25) (layer F.Cu) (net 6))
 (segment (start 198.1736 151.94999) (end 175.514291 151.94999) (width 0.25) (layer F.Cu) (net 6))
 (segment (start 175.514291 151.94999) (end 168.91 145.345699) (width 0.25) (layer F.Cu) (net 6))
 (segment (start 200.555001 149.568589) (end 198.1736 151.94999) (width 0.25) (layer F.Cu) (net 6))
 (segment (start 157.8 111.44) (end 168.91 122.55) (width 0.25) (layer B.Cu) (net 6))
 (segment (start 200.555001 144.255001) (end 200.555001 149.568589) (width 0.25) (layer F.Cu) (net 6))
 (segment (start 199.48 143.18) (end 200.555001 144.255001) (width 0.25) (layer F.Cu) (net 6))
 (via (at 168.91 132.08) (size 0.8) (drill 0.4) (layers F.Cu B.Cu) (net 6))
 (segment (start 198.12 149.86) (end 195.58 149.86) (width 0.25) (layer F.Cu) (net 9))
 (segment (start 199.48 148.5) (end 198.12 149.86) (width 0.25) (layer F.Cu) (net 9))
 (segment (start 199.48 146.38) (end 199.48 148.5) (width 0.25) (layer F.Cu) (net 9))
 (segment (start 171.45 102.87) (end 167.64 102.87) (width 0.25) (layer F.Cu) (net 8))
 (segment (start 167.55 102.96) (end 167.64 102.87) (width 0.25) (layer F.Cu) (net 8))
 (segment (start 167.55 108.89) (end 167.55 102.96) (width 0.25) (layer F.Cu) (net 8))
 (segment (start 128.27 118.11) (end 139.7 106.68) (width 0.25) (layer F.Cu) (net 3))
 (segment (start 124.174366 118.11) (end 128.27 118.11) (width 0.25) (layer F.Cu) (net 3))
 (segment (start 123.19 117.125634) (end 124.174366 118.11) (width 0.25) (layer F.Cu) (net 3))
 (segment (start 123.19 115.57) (end 123.19 117.125634) (width 0.25) (layer F.Cu) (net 3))
 (segment (start 139.8925 106.68) (end 139.7 106.68) (width 0.25) (layer F.Cu) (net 3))
 (segment (start 144.78 101.7925) (end 139.8925 106.68) (width 0.25) (layer F.Cu) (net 3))
 (segment (start 123.19 121.92) (end 123.19 115.57) (width 0.25) (layer B.Cu) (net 3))
 (segment (start 157.48 156.21) (end 123.19 121.92) (width 0.25) (layer B.Cu) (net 3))
 (segment (start 171.45 156.21) (end 157.48 156.21) (width 0.25) (layer B.Cu) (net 3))
 (segment (start 212.09 107.95) (end 212.09 96.52) (width 0.25) (layer B.Cu) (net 3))
 (segment (start 212.09 96.52) (end 198.12 82.55) (width 0.25) (layer B.Cu) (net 3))
 (via (at 149.86 93.98) (size 0.8) (drill 0.4) (layers F.Cu B.Cu) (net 3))
 (segment (start 161.29 82.55) (end 149.86 93.98) (width 0.25) (layer B.Cu) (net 3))
 (segment (start 148.59 100.33) (end 147.1275 101.7925) (width 0.25) (layer F.Cu) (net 3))
 (segment (start 148.59 95.25) (end 148.59 100.33) (width 0.25) (layer F.Cu) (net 3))
 (segment (start 147.1275 101.7925) (end 144.78 101.7925) (width 0.25) (layer F.Cu) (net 3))
 (segment (start 149.86 93.98) (end 148.59 95.25) (width 0.25) (layer F.Cu) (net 3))
 (segment (start 193.04 82.55) (end 161.29 82.55) (width 0.25) (layer B.Cu) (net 3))
 (segment (start 198.12 82.55) (end 193.04 82.55) (width 0.25) (layer B.Cu) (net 3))
 (segment (start 193.04 86.36) (end 193.04 82.55) (width 0.25) (layer B.Cu) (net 3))
 (segment (start 173.99 105.41) (end 193.04 86.36) (width 0.25) (layer B.Cu) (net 3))
 (segment (start 171.45 105.41) (end 173.99 105.41) (width 0.25) (layer B.Cu) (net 3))
 (segment (start 163.83 80.01) (end 161.29 82.55) (width 0.25) (layer B.Cu) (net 3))
 (segment (start 163.83 67.31) (end 163.83 80.01) (width 0.25) (layer B.Cu) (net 3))
 (segment (start 137.874999 111.665001) (end 144.13 105.41) (width 0.25) (layer F.Cu) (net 2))
 (segment (start 137.874999 125.174999) (end 137.874999 111.665001) (width 0.25) (layer F.Cu) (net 2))
 (segment (start 139.7 127) (end 137.874999 125.174999) (width 0.25) (layer F.Cu) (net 2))
 (segment (start 148.46 109.39) (end 148.91 109.84) (width 0.25) (layer F.Cu) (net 7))
 (segment (start 148.46 105.41) (end 148.46 109.39) (width 0.25) (layer F.Cu) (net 7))
 (segment (start 148.61 111.44) (end 148.91 111.14) (width 0.25) (layer F.Cu) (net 7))
 (segment (start 146.05 111.44) (end 148.61 111.44) (width 0.25) (layer F.Cu) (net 7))
 (segment (start 145.43 105.41) (end 148.46 105.41) (width 0.25) (layer F.Cu) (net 7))
 (segment (start 153.67 127) (end 153.67 121.92) (width 0.25) (layer F.Cu) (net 7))
 (segment (start 146.05 114.3) (end 146.05 111.44) (width 0.25) (layer F.Cu) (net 7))
 (segment (start 153.67 121.92) (end 146.05 114.3) (width 0.25) (layer F.Cu) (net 7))
 (segment (start 134.62 147.56625) (end 134.62 145.63) (width 0.25) (layer F.Cu) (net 13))
 (segment (start 135.64375 148.59) (end 134.62 147.56625) (width 0.25) (layer F.Cu) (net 13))
 (segment (start 134.62 145.63) (end 137.07 143.18) (width 0.25) (layer F.Cu) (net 13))
 (segment (start 137.562501 148.59) (end 135.64375 148.59) (width 0.25) (layer F.Cu) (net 13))
 (segment (start 162.65 123.502501) (end 137.562501 148.59) (width 0.25) (layer F.Cu) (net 13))
 (segment (start 162.65 112.09) (end 162.65 123.502501) (width 0.25) (layer F.Cu) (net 13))
 (via (at 135.89 73.66) (size 0.8) (drill 0.4) (layers F.Cu B.Cu) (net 12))
 (segment (start 135.89 73.66) (end 137.16 73.66) (width 0.25) (layer B.Cu) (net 12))
 (via (at 139.7 76.2) (size 0.8) (drill 0.4) (layers F.Cu B.Cu) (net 12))
 (segment (start 137.16 73.66) (end 139.7 76.2) (width 0.25) (layer B.Cu) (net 12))
 (segment (start 138.76 77.14) (end 137.07 77.14) (width 0.25) (layer F.Cu) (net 12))
 (segment (start 139.7 76.2) (end 138.76 77.14) (width 0.25) (layer F.Cu) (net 12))
 (segment (start 132.314261 73.66) (end 135.89 73.66) (width 0.25) (layer F.Cu) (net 12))
 (segment (start 128.27 77.704261) (end 132.314261 73.66) (width 0.25) (layer F.Cu) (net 12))
 (segment (start 128.27 88.792346) (end 128.27 77.704261) (width 0.25) (layer F.Cu) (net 12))
 (segment (start 116.84 123.19) (end 116.84 100.222346) (width 0.25) (layer F.Cu) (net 12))
 (segment (start 123.19 137.08823) (end 123.19 129.54) (width 0.25) (layer F.Cu) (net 12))
 (segment (start 116.84 100.222346) (end 128.27 88.792346) (width 0.25) (layer F.Cu) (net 12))
 (segment (start 131.14 145.03823) (end 123.19 137.08823) (width 0.25) (layer F.Cu) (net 12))
 (segment (start 123.19 129.54) (end 116.84 123.19) (width 0.25) (layer F.Cu) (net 12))
 (segment (start 131.14 146.38) (end 131.14 145.03823) (width 0.25) (layer F.Cu) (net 12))
 (segment (start 132.17 146.38) (end 131.14 146.38) (width 0.25) (layer F.Cu) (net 12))
 (segment (start 132.17 79.59) (end 148.649276 63.110724) (width 0.25) (layer F.Cu) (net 11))
 (segment (start 132.17 80.34) (end 132.17 79.59) (width 0.25) (layer F.Cu) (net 11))
 (segment (start 203.11 77.14) (end 203.11 76.11) (width 0.25) (layer F.Cu) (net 11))
 (segment (start 203.11 76.11) (end 194.31 67.31) (width 0.25) (layer F.Cu) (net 11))
 (segment (start 194.31 67.31) (end 182.388552 67.31) (width 0.25) (layer F.Cu) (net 11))
 (segment (start 182.388552 67.31) (end 178.189276 63.110724) (width 0.25) (layer F.Cu) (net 11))
 (segment (start 148.649276 63.110724) (end 178.189276 63.110724) (width 0.25) (layer F.Cu) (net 11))
 (segment (start 198.21 80.34) (end 204.47 86.6) (width 0.25) (layer F.Cu) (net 10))
 (segment (start 204.47 143.09) (end 204.38 143.18) (width 0.25) (layer F.Cu) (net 10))
 (segment (start 204.47 86.6) (end 204.47 143.09) (width 0.25) (layer F.Cu) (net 10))
 (segment (start 150.81 109.84) (end 151.78 109.84) (width 0.25) (layer F.Cu) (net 5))
 (segment (start 151.78 109.84) (end 153.67 107.95) (width 0.25) (layer F.Cu) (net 5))
 (segment (start 153.67 107.95) (end 153.67 106.68) (width 0.25) (layer F.Cu) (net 5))
 (segment (start 152.4 105.41) (end 151.26 105.41) (width 0.25) (layer F.Cu) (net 5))
 (segment (start 153.67 106.68) (end 152.4 105.41) (width 0.25) (layer F.Cu) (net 5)))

